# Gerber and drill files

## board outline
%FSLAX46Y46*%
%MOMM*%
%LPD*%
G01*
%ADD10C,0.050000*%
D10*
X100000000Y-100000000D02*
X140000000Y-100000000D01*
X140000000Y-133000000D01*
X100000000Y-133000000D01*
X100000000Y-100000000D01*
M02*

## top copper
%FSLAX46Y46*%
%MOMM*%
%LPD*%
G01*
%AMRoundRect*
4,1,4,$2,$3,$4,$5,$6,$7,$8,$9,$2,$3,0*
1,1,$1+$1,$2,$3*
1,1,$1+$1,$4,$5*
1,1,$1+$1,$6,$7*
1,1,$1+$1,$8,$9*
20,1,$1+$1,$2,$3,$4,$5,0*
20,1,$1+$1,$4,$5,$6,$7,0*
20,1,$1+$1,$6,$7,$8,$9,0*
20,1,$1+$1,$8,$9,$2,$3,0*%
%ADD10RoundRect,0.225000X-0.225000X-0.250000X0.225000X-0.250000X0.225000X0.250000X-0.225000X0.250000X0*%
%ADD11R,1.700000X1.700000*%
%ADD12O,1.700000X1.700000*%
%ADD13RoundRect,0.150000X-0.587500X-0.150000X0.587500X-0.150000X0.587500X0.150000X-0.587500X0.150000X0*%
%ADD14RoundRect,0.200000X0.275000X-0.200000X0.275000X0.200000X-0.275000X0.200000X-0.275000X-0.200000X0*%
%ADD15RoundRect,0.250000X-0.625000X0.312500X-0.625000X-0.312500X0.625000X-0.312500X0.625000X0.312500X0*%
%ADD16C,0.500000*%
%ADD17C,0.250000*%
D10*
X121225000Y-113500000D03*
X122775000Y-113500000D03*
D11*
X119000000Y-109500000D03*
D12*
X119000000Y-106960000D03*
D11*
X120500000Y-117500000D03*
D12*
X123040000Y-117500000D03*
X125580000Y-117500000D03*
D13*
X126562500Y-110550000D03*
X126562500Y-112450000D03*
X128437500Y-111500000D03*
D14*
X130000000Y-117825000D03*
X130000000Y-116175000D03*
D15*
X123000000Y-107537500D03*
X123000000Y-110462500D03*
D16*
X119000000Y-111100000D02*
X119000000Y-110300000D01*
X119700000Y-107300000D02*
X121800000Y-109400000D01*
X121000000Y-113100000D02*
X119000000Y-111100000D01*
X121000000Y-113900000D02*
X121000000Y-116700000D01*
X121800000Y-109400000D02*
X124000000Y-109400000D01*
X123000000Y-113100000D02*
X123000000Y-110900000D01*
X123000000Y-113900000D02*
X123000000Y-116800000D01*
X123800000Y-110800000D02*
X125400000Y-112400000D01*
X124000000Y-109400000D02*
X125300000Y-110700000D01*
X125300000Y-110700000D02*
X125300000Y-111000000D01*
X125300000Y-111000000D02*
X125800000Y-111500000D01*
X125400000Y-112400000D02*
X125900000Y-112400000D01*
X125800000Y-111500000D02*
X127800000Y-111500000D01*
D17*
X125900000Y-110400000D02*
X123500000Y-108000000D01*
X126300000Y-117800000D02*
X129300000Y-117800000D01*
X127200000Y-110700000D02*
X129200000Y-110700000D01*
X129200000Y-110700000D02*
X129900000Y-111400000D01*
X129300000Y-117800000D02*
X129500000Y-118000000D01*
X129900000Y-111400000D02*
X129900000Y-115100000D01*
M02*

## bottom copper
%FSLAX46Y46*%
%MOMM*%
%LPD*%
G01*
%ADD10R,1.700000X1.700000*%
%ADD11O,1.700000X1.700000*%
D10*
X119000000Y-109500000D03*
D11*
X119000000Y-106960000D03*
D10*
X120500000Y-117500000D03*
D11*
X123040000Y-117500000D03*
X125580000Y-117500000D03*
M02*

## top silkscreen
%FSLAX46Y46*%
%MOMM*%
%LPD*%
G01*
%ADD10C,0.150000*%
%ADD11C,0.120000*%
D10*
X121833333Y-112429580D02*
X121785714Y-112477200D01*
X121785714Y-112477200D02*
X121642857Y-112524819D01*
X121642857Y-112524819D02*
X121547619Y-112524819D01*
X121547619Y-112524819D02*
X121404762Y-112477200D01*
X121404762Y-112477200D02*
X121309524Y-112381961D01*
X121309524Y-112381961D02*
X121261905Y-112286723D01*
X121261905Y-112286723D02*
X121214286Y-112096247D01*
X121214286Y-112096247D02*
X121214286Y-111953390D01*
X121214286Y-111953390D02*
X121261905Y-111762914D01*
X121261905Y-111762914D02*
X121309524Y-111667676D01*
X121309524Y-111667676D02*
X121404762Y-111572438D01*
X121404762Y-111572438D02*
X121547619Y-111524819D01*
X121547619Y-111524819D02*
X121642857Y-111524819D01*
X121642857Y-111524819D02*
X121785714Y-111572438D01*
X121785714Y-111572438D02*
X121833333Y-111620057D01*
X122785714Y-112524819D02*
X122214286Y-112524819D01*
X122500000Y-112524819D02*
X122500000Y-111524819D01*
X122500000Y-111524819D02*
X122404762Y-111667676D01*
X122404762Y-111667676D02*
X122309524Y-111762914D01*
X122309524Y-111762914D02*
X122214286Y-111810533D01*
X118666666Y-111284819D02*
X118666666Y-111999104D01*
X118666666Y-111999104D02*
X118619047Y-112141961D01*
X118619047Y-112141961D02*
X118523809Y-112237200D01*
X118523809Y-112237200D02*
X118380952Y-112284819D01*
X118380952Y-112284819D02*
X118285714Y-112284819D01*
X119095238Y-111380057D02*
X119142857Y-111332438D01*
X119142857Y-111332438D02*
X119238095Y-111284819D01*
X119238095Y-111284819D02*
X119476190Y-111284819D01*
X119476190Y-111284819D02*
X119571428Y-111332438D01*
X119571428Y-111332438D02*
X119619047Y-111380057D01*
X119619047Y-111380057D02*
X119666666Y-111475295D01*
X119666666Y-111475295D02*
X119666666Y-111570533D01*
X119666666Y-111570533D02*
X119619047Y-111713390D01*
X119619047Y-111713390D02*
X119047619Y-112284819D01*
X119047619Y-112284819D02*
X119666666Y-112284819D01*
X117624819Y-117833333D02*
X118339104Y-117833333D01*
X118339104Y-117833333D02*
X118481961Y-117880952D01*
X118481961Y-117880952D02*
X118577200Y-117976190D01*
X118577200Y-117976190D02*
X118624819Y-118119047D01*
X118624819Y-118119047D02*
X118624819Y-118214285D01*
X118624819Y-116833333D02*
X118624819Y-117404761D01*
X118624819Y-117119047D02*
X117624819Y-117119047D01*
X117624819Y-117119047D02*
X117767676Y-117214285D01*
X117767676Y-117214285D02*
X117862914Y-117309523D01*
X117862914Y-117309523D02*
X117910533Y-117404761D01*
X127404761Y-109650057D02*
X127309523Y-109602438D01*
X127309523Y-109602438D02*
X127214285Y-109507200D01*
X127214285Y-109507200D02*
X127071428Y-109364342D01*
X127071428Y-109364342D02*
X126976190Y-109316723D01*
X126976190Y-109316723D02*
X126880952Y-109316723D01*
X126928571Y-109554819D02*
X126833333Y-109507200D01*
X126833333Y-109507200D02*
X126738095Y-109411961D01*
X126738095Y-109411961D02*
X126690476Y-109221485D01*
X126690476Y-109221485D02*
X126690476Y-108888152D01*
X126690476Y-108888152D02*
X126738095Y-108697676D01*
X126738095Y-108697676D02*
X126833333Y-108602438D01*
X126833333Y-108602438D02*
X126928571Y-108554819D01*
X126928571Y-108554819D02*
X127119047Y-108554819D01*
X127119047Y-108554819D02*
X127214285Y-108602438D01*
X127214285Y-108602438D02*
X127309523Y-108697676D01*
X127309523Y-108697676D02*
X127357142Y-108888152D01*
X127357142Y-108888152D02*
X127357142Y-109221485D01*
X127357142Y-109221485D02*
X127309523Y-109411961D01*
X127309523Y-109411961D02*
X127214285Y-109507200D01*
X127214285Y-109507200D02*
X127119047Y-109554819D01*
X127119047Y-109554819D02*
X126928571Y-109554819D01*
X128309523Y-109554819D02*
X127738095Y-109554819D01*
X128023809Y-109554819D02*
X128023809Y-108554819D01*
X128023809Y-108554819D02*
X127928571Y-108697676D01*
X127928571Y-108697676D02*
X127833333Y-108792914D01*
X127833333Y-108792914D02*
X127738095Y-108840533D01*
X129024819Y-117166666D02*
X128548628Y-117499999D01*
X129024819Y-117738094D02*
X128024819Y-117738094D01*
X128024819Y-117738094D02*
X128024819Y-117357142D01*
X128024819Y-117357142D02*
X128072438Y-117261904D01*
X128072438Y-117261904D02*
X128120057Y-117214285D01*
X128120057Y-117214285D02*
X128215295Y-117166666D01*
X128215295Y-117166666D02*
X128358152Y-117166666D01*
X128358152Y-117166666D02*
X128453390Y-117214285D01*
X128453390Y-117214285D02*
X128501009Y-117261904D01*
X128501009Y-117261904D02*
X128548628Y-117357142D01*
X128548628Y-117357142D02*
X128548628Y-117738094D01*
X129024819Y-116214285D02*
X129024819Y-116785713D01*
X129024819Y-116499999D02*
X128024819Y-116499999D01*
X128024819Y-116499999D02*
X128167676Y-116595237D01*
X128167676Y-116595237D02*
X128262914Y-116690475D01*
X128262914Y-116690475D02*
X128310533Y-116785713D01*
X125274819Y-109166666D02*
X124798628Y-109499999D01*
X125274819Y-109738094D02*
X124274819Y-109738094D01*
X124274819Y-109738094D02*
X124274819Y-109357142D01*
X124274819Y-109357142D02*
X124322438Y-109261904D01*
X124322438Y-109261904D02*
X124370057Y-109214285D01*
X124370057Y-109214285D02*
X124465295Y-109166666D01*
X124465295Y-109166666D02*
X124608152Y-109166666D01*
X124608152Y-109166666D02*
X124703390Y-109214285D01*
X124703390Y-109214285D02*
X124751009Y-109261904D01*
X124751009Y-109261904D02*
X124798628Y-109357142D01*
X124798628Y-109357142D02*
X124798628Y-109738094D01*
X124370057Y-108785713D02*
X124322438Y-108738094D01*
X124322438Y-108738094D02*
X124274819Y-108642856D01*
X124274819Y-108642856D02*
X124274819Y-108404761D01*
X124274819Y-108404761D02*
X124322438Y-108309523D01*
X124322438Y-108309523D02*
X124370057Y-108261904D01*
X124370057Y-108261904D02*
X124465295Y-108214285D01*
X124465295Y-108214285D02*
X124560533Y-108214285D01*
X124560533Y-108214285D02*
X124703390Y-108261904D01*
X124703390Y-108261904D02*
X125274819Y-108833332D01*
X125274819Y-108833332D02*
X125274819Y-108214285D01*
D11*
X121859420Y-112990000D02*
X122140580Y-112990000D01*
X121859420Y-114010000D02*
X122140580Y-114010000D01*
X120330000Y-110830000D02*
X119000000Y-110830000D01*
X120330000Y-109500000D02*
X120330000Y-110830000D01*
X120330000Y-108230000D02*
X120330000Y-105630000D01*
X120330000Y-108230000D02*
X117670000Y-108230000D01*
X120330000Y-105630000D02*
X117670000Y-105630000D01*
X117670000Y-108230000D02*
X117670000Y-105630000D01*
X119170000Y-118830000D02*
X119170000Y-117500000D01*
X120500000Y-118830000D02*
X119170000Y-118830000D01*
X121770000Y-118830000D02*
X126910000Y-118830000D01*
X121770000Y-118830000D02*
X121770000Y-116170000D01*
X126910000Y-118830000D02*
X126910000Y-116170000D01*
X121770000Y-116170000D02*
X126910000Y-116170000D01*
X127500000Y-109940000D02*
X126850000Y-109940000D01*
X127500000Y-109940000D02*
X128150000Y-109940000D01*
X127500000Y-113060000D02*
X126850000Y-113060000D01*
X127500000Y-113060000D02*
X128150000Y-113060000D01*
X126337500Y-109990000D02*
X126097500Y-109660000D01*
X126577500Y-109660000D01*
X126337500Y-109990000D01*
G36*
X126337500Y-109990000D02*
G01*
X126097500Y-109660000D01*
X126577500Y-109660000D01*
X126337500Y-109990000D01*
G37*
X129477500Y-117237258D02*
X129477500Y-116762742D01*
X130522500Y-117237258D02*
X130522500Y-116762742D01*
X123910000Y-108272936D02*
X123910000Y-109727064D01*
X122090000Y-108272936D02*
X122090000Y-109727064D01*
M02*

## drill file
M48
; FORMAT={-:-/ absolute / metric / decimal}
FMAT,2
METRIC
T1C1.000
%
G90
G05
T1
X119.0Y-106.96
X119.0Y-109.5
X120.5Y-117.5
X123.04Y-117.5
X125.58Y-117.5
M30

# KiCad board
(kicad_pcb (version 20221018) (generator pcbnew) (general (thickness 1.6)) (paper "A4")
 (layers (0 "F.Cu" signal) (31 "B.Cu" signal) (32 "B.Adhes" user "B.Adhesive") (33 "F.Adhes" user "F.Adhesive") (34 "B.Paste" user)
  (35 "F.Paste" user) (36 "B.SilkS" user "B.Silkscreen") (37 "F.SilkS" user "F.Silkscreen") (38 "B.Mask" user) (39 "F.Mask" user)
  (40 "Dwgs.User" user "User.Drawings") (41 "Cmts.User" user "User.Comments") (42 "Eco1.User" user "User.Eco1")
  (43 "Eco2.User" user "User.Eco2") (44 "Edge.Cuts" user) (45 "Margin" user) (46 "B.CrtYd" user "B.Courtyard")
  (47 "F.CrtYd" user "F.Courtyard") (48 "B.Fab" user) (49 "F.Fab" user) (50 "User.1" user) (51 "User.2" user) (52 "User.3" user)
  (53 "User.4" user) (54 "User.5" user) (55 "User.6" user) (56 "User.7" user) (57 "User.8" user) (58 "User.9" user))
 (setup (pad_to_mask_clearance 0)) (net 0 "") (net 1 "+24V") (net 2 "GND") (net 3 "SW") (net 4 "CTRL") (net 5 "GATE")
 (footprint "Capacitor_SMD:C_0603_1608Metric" (layer "F.Cu") (at 122 113.5)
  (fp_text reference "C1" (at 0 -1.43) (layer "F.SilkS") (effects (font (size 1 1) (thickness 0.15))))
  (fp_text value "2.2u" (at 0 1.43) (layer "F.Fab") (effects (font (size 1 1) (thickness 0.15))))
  (fp_line (start -0.14058 -0.51) (end 0.14058 -0.51) (stroke (width 0.12) (type solid)) (layer "F.SilkS"))
  (fp_line (start -0.14058 0.51) (end 0.14058 0.51) (stroke (width 0.12) (type solid)) (layer "F.SilkS"))
  (pad "1" smd roundrect (at -0.775 0) (size 0.9 0.95) (layers "F.Cu" "F.Paste" "F.Mask") (roundrect_rratio 0.25) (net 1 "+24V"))
  (pad "2" smd roundrect (at 0.775 0) (size 0.9 0.95) (layers "F.Cu" "F.Paste" "F.Mask") (roundrect_rratio 0.25) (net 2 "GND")))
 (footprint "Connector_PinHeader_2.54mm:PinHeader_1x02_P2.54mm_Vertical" (layer "F.Cu") (at 119 109.5 180)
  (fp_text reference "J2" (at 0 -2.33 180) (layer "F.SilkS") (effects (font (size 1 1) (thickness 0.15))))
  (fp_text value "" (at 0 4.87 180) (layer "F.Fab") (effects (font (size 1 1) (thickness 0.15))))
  (fp_line (start -1.33 -1.33) (end 0 -1.33) (stroke (width 0.12) (type solid)) (layer "F.SilkS"))
  (fp_line (start -1.33 0) (end -1.33 -1.33) (stroke (width 0.12) (type solid)) (layer "F.SilkS"))
  (fp_line (start -1.33 1.27) (end -1.33 3.87) (stroke (width 0.12) (type solid)) (layer "F.SilkS"))
  (fp_line (start -1.33 1.27) (end 1.33 1.27) (stroke (width 0.12) (type solid)) (layer "F.SilkS"))
  (fp_line (start -1.33 3.87) (end 1.33 3.87) (stroke (width 0.12) (type solid)) (layer "F.SilkS"))
  (fp_line (start 1.33 1.27) (end 1.33 3.87) (stroke (width 0.12) (type solid)) (layer "F.SilkS"))
  (pad "1" thru_hole rect (at 0 0 180) (size 1.7 1.7) (drill 1) (layers "*.Cu" "*.Mask") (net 1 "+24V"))
  (pad "2" thru_hole oval (at 0 2.54 180) (size 1.7 1.7) (drill 1) (layers "*.Cu" "*.Mask") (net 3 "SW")))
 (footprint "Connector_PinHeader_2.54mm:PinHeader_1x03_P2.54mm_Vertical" (layer "F.Cu") (at 120.5 117.5 90)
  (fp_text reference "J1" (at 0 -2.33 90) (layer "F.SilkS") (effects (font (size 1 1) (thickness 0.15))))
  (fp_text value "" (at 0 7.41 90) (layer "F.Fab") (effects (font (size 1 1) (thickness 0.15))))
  (fp_line (start -1.33 -1.33) (end 0 -1.33) (stroke (width 0.12) (type solid)) (layer "F.SilkS"))
  (fp_line (start -1.33 0) (end -1.33 -1.33) (stroke (width 0.12) (type solid)) (layer "F.SilkS"))
  (fp_line (start -1.33 1.27) (end -1.33 6.41) (stroke (width 0.12) (type solid)) (layer "F.SilkS"))
  (fp_line (start -1.33 1.27) (end 1.33 1.27) (stroke (width 0.12) (type solid)) (layer "F.SilkS"))
  (fp_line (start -1.33 6.41) (end 1.33 6.41) (stroke (width 0.12) (type solid)) (layer "F.SilkS"))
  (fp_line (start 1.33 1.27) (end 1.33 6.41) (stroke (width 0.12) (type solid)) (layer "F.SilkS"))
  (pad "1" thru_hole rect (at 0 0 90) (size 1.7 1.7) (drill 1) (layers "*.Cu" "*.Mask") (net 1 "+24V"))
  (pad "2" thru_hole oval (at 0 2.54 90) (size 1.7 1.7) (drill 1) (layers "*.Cu" "*.Mask") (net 2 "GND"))
  (pad "3" thru_hole oval (at 0 5.08 90) (size 1.7 1.7) (drill 1) (layers "*.Cu" "*.Mask") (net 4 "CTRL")))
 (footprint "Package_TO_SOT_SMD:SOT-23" (layer "F.Cu") (at 127.5 111.5)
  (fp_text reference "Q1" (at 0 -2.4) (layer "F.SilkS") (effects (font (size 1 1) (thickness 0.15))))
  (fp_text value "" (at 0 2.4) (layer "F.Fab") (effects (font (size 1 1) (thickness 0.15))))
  (fp_line (start 0 -1.56) (end -0.65 -1.56) (stroke (width 0.12) (type solid)) (layer "F.SilkS"))
  (fp_line (start 0 -1.56) (end 0.65 -1.56) (stroke (width 0.12) (type solid)) (layer "F.SilkS"))
  (fp_line (start 0 1.56) (end -0.65 1.56) (stroke (width 0.12) (type solid)) (layer "F.SilkS"))
  (fp_line (start 0 1.56) (end 0.65 1.56) (stroke (width 0.12) (type solid)) (layer "F.SilkS"))
  (fp_poly
   (pts (xy -1.1625 -1.51) (xy -1.4025 -1.84) (xy -0.9225 -1.84) (xy -1.1625 -1.51)) (stroke (width 0.12) (type solid)) (fill solid)
   (layer "F.SilkS"))
  (pad "1" smd roundrect (at -0.9375 -0.95) (size 1.475 0.6) (layers "F.Cu" "F.Paste" "F.Mask") (roundrect_rratio 0.25) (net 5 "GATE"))
  (pad "2" smd roundrect (at -0.9375 0.95) (size 1.475 0.6) (layers "F.Cu" "F.Paste" "F.Mask") (roundrect_rratio 0.25) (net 2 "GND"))
  (pad "3" smd roundrect (at 0.9375 0) (size 1.475 0.6) (layers "F.Cu" "F.Paste" "F.Mask") (roundrect_rratio 0.25) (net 3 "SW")))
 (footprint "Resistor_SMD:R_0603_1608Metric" (layer "F.Cu") (at 130 117 90)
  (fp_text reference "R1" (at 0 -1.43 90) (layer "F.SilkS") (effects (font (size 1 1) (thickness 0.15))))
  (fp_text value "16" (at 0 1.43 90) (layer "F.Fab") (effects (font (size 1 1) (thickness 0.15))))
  (fp_line (start -0.237258 -0.5225) (end 0.237258 -0.5225) (stroke (width 0.12) (type solid)) (layer "F.SilkS"))
  (fp_line (start -0.237258 0.5225) (end 0.237258 0.5225) (stroke (width 0.12) (type solid)) (layer "F.SilkS"))
  (pad "1" smd roundrect (at -0.825 0 90) (size 0.8 0.95) (layers "F.Cu" "F.Paste" "F.Mask") (roundrect_rratio 0.25) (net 4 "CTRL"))
  (pad "2" smd roundrect (at 0.825 0 90) (size 0.8 0.95) (layers "F.Cu" "F.Paste" "F.Mask") (roundrect_rratio 0.25) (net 5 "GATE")))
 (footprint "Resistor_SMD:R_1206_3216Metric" (layer "F.Cu") (at 123 109 -90)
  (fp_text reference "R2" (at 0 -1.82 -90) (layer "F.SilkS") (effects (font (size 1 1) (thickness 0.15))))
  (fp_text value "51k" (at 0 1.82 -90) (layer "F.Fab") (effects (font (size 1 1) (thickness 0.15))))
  (fp_line (start -0.727064 -0.91) (end 0.727064 -0.91) (stroke (width 0.12) (type solid)) (layer "F.SilkS"))
  (fp_line (start -0.727064 0.91) (end 0.727064 0.91) (stroke (width 0.12) (type solid)) (layer "F.SilkS"))
  (pad "1" smd roundrect (at -1.4625 0 270) (size 1.125 1.75) (layers "F.Cu" "F.Paste" "F.Mask") (roundrect_rratio 0.222222) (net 5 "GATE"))
  (pad "2" smd roundrect (at 1.4625 0 270) (size 1.125 1.75) (layers "F.Cu" "F.Paste" "F.Mask") (roundrect_rratio 0.222222) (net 2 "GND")))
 (gr_rect (start 100 100) (end 140 133) (stroke (width 0.05) (type default)) (fill none) (layer "Edge.Cuts"))
 (segment (start 119 111.1) (end 119 110.3) (width 0.5) (layer "F.Cu") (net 1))
 (segment (start 119.7 107.3) (end 121.8 109.4) (width 0.5) (layer "F.Cu") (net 3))
 (segment (start 121 113.1) (end 119 111.1) (width 0.5) (layer "F.Cu") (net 1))
 (segment (start 121 113.9) (end 121 116.7) (width 0.5) (layer "F.Cu") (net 1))
 (segment (start 121.8 109.4) (end 124 109.4) (width 0.5) (layer "F.Cu") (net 3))
 (segment (start 123 113.1) (end 123 110.9) (width 0.5) (layer "F.Cu") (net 2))
 (segment (start 123 113.9) (end 123 116.8) (width 0.5) (layer "F.Cu") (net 2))
 (segment (start 123.8 110.8) (end 125.4 112.4) (width 0.5) (layer "F.Cu") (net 2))
 (segment (start 124 109.4) (end 125.3 110.7) (width 0.5) (layer "F.Cu") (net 3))
 (segment (start 125.3 110.7) (end 125.3 111) (width 0.5) (layer "F.Cu") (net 3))
 (segment (start 125.3 111) (end 125.8 111.5) (width 0.5) (layer "F.Cu") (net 3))
 (segment (start 125.4 112.4) (end 125.9 112.4) (width 0.5) (layer "F.Cu") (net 2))
 (segment (start 125.8 111.5) (end 127.8 111.5) (width 0.5) (layer "F.Cu") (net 3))
 (segment (start 125.9 110.4) (end 123.5 108) (width 0.25) (layer "F.Cu") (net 5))
 (segment (start 126.3 117.8) (end 129.3 117.8) (width 0.25) (layer "F.Cu") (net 4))
 (segment (start 127.2 110.7) (end 129.2 110.7) (width 0.25) (layer "F.Cu") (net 5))
 (segment (start 129.2 110.7) (end 129.9 111.4) (width 0.25) (layer "F.Cu") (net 5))
 (segment (start 129.3 117.8) (end 129.5 118) (width 0.25) (layer "F.Cu") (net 4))
 (segment (start 129.9 111.4) (end 129.9 115.1) (width 0.25) (layer "F.Cu") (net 5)))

